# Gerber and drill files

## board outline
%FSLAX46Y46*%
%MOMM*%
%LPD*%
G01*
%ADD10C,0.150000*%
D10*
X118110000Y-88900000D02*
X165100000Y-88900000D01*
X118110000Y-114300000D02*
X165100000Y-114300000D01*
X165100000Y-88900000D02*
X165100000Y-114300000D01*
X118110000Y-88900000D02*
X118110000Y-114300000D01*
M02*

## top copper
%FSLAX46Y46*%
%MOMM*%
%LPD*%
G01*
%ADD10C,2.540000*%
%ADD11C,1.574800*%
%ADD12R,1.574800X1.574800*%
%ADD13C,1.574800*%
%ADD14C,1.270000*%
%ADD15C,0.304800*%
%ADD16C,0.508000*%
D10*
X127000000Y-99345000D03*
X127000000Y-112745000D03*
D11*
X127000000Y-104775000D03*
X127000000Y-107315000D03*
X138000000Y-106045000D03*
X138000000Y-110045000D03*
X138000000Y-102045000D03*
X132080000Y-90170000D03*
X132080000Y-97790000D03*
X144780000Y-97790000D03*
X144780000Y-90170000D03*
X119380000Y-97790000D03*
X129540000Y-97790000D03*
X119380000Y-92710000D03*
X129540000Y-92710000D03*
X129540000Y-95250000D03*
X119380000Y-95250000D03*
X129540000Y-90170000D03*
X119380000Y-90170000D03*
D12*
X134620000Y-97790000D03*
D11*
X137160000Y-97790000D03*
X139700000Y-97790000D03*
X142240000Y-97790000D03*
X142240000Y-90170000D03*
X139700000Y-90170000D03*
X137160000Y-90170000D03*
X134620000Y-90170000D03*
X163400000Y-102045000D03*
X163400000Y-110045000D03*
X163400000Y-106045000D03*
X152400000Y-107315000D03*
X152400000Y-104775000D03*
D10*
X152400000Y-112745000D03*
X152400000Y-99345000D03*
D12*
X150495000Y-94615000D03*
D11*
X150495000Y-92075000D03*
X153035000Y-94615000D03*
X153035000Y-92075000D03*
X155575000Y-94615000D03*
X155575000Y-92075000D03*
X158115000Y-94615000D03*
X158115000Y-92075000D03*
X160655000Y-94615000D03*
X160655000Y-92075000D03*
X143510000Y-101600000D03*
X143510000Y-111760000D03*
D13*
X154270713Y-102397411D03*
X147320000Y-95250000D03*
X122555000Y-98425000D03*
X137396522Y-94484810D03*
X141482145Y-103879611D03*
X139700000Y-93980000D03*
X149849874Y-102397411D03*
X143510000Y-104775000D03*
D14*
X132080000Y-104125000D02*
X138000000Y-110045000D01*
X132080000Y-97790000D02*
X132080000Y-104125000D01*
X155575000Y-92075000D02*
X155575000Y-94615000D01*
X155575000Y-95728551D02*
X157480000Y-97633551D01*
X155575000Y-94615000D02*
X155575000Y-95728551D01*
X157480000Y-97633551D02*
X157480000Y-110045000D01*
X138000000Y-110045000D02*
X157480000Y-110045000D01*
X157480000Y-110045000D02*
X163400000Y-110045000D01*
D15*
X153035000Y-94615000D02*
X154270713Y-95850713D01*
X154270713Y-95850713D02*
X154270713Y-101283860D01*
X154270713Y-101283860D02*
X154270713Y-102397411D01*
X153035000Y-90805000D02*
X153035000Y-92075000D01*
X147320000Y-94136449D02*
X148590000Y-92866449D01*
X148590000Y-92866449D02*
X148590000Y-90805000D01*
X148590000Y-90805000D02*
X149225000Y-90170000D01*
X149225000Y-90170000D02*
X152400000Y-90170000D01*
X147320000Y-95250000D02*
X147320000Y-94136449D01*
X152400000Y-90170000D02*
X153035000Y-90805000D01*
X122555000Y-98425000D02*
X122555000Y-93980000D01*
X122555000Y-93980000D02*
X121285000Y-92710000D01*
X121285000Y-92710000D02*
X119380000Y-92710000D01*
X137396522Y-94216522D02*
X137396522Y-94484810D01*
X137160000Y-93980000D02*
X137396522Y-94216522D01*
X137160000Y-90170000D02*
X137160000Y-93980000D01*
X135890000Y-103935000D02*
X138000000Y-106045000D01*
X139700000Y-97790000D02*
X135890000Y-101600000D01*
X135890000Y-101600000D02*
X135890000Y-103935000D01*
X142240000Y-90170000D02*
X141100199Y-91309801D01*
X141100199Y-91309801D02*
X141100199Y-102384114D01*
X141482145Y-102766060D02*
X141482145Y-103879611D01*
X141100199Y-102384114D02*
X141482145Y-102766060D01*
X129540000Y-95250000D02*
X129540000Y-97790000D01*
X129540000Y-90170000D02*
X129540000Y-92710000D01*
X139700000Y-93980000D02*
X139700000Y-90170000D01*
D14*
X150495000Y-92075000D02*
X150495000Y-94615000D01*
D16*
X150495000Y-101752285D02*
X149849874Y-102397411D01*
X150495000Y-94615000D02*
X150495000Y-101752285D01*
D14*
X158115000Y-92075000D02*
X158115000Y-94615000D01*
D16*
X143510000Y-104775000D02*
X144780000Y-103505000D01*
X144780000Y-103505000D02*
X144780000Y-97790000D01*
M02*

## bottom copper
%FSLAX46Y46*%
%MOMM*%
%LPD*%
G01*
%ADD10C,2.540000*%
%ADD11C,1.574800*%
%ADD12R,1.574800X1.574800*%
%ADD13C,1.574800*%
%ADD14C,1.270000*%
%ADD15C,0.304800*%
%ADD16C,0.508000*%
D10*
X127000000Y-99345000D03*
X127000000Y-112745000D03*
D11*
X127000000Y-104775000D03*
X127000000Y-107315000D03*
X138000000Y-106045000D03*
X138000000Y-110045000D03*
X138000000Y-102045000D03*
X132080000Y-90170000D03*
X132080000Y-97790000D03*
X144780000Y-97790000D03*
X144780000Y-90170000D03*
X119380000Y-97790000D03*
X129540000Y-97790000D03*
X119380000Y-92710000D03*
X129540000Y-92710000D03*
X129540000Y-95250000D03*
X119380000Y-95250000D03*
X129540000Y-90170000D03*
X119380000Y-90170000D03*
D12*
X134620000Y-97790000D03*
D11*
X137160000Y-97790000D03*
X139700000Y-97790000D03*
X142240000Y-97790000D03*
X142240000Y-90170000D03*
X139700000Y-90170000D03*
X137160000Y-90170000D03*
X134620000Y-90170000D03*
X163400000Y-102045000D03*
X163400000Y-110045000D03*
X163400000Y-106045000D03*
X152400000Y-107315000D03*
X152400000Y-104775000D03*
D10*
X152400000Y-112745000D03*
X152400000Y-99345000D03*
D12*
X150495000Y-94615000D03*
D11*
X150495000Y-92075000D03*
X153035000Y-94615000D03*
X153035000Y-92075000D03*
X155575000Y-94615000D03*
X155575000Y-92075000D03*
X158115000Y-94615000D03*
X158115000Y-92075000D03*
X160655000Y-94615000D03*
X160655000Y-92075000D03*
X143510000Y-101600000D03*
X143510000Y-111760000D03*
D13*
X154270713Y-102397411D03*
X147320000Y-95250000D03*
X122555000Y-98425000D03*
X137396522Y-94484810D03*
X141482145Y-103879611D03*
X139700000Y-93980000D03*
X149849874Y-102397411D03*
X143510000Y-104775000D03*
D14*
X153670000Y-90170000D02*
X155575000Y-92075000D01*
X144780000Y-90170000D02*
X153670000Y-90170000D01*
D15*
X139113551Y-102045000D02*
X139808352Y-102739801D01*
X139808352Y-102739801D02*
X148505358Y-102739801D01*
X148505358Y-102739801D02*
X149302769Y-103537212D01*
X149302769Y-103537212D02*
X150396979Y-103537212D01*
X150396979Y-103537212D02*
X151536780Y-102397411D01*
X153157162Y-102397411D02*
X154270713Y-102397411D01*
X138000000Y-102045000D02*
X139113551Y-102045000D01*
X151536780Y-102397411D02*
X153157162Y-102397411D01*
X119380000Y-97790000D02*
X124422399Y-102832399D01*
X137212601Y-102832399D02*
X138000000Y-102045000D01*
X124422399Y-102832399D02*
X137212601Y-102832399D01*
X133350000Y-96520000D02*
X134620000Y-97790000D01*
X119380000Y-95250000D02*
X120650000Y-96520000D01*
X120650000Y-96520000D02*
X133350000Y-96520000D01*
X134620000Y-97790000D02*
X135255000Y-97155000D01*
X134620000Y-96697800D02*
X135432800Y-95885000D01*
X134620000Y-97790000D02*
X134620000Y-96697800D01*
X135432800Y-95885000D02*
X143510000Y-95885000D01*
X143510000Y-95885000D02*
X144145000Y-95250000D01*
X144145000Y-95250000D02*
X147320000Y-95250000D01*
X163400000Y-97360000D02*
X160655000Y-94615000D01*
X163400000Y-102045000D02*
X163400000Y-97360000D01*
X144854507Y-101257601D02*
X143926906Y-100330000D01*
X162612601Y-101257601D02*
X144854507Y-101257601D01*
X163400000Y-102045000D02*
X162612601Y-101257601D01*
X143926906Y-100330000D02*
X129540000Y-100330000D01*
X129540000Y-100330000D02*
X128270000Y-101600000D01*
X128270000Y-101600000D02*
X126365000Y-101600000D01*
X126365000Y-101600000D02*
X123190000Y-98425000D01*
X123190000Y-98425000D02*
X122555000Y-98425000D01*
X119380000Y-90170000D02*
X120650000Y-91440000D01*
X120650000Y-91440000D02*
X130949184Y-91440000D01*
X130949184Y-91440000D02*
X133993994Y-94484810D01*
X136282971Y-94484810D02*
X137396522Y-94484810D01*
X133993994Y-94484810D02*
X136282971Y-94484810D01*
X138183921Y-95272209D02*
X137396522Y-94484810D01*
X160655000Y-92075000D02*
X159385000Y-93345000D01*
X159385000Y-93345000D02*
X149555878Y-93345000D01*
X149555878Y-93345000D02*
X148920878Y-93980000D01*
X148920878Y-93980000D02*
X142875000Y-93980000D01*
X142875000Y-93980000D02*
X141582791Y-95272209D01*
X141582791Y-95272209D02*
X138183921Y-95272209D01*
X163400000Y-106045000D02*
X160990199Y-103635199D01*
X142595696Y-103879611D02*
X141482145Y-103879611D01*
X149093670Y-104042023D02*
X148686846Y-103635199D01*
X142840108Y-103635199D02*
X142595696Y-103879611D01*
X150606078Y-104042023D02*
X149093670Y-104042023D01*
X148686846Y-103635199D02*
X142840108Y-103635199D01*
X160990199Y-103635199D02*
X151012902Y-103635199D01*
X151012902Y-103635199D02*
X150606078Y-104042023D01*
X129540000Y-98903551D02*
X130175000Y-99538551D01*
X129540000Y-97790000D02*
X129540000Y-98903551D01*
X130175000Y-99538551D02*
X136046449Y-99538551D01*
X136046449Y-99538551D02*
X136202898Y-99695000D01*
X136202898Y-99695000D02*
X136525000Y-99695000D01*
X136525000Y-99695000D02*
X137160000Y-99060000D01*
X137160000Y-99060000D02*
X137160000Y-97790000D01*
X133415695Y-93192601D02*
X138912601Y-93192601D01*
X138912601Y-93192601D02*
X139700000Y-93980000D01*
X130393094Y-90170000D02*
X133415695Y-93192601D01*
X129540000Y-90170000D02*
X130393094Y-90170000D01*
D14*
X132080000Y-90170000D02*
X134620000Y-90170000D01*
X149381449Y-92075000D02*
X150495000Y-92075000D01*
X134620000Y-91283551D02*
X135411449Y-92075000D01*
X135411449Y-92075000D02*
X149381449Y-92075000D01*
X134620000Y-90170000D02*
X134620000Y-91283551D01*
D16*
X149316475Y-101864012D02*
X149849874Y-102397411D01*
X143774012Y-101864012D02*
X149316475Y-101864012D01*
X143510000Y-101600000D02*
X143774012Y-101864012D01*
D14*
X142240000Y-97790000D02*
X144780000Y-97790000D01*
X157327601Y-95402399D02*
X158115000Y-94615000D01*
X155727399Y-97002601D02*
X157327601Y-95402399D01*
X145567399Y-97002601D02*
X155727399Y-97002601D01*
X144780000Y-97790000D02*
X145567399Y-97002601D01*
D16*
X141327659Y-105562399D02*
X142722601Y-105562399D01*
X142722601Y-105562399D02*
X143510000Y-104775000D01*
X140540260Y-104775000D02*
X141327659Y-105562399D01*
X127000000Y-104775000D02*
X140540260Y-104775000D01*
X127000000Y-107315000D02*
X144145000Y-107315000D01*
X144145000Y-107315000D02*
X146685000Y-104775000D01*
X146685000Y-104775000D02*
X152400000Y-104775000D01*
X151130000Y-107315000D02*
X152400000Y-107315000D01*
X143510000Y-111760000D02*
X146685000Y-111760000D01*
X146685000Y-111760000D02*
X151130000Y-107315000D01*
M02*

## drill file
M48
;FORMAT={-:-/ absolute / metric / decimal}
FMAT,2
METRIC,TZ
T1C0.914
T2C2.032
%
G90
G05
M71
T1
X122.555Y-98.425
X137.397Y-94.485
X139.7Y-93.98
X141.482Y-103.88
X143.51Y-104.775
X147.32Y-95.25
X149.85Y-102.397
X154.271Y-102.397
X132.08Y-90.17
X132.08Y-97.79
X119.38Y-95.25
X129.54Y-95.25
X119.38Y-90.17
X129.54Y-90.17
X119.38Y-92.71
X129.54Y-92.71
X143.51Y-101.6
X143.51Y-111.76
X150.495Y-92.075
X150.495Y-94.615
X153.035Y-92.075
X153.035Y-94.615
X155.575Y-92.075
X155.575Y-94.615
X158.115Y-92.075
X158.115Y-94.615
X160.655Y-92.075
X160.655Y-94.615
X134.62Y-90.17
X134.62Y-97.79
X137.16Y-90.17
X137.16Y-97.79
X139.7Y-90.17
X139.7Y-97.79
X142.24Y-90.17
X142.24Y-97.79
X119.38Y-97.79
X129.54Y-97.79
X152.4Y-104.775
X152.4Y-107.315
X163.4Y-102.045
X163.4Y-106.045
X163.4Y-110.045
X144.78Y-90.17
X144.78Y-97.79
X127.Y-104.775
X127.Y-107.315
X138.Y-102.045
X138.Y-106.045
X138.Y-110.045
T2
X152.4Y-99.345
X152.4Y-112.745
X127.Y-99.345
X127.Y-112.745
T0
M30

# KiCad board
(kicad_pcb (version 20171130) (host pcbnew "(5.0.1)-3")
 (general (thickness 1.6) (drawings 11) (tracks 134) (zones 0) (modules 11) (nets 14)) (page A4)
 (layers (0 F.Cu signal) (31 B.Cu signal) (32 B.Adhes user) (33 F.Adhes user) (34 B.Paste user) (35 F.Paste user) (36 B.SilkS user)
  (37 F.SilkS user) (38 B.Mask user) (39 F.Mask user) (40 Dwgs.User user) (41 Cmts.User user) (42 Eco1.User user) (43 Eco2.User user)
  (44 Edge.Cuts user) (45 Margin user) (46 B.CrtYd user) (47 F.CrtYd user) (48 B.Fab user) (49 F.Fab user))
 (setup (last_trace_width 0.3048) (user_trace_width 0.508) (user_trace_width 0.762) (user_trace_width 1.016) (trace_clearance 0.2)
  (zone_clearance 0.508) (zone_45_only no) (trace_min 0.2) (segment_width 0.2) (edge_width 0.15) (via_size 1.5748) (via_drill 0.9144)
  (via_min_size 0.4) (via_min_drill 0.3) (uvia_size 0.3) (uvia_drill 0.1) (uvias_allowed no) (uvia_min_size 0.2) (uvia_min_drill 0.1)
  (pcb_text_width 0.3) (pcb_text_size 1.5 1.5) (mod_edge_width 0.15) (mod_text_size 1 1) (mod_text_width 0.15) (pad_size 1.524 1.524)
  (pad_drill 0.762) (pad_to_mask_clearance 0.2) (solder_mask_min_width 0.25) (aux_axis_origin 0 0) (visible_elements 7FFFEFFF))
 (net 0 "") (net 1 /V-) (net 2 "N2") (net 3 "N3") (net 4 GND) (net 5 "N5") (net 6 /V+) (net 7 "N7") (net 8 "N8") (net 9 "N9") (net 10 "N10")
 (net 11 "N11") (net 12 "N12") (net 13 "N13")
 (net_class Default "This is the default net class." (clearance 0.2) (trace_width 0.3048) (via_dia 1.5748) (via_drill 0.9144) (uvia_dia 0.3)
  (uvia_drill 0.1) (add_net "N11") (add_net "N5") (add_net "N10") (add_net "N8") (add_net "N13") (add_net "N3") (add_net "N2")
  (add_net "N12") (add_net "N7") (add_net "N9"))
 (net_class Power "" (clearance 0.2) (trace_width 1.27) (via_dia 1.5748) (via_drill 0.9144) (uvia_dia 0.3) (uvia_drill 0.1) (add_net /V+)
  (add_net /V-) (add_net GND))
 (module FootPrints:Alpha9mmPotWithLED (layer B.Cu) (at 127 106.045 270)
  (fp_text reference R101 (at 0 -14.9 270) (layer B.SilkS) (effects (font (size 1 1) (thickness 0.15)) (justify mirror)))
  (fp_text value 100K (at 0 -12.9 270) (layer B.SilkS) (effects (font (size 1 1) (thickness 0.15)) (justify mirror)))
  (pad "" thru_hole circle (at -6.7 0 270) (size 2.54 2.54) (drill 2.032) (layers *.Cu *.Mask B.SilkS))
  (pad "" thru_hole circle (at 6.7 0 270) (size 2.54 2.54) (drill 2.032) (layers *.Cu *.Mask B.SilkS))
  (pad 4 thru_hole circle (at -1.27 0 270) (size 1.5748 1.5748) (drill 0.9144) (layers *.Cu *.Mask B.SilkS) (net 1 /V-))
  (pad 5 thru_hole circle (at 1.27 0 270) (size 1.5748 1.5748) (drill 0.9144) (layers *.Cu *.Mask B.SilkS) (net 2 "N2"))
  (pad 2 thru_hole circle (at 0 -11 270) (size 1.5748 1.5748) (drill 0.9144) (layers *.Cu *.Mask B.SilkS) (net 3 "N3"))
  (pad 3 thru_hole circle (at 4 -11 270) (size 1.5748 1.5748) (drill 0.9144) (layers *.Cu *.Mask B.SilkS) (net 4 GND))
  (pad 1 thru_hole circle (at -4 -11 270) (size 1.5748 1.5748) (drill 0.9144) (layers *.Cu *.Mask B.SilkS) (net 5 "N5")))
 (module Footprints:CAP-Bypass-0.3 (layer F.Cu) (at 132.08 93.98 270)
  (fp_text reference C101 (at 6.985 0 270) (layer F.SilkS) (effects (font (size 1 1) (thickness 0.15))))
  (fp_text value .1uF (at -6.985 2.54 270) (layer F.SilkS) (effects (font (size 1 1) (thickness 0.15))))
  (pad 1 thru_hole circle (at -3.81 0 270) (size 1.5748 1.5748) (drill 0.9144) (layers *.Cu *.Mask F.SilkS) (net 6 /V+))
  (pad 2 thru_hole circle (at 3.81 0 270) (size 1.5748 1.5748) (drill 0.9144) (layers *.Cu *.Mask F.SilkS) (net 4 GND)))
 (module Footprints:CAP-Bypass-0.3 (layer F.Cu) (at 144.78 93.98 90)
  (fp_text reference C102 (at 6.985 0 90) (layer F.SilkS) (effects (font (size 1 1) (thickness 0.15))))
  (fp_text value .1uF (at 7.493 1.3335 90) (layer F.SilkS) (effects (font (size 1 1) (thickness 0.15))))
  (pad 1 thru_hole circle (at -3.81 0 90) (size 1.5748 1.5748) (drill 0.9144) (layers *.Cu *.Mask F.SilkS) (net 1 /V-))
  (pad 2 thru_hole circle (at 3.81 0 90) (size 1.5748 1.5748) (drill 0.9144) (layers *.Cu *.Mask F.SilkS) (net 4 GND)))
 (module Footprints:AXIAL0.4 (layer F.Cu) (at 124.46 97.79)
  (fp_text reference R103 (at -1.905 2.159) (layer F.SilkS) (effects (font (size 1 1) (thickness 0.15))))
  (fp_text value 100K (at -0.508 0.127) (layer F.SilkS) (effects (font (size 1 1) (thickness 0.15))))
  (pad 1 thru_hole circle (at -5.08 0) (size 1.5748 1.5748) (drill 0.9144) (layers *.Cu *.Mask F.SilkS) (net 5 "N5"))
  (pad 2 thru_hole circle (at 5.08 0) (size 1.5748 1.5748) (drill 0.9144) (layers *.Cu *.Mask F.SilkS) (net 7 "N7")))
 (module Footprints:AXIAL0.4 (layer F.Cu) (at 124.46 92.71)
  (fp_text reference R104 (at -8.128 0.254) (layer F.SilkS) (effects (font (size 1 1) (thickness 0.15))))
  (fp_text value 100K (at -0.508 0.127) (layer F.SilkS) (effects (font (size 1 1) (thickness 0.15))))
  (pad 1 thru_hole circle (at -5.08 0) (size 1.5748 1.5748) (drill 0.9144) (layers *.Cu *.Mask F.SilkS) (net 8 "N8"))
  (pad 2 thru_hole circle (at 5.08 0) (size 1.5748 1.5748) (drill 0.9144) (layers *.Cu *.Mask F.SilkS) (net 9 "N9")))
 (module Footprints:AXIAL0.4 (layer F.Cu) (at 124.46 95.25 180)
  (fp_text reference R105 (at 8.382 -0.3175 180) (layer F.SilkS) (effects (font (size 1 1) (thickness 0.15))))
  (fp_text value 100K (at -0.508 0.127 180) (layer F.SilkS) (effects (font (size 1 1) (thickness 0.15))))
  (pad 1 thru_hole circle (at -5.08 0 180) (size 1.5748 1.5748) (drill 0.9144) (layers *.Cu *.Mask F.SilkS) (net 7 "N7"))
  (pad 2 thru_hole circle (at 5.08 0 180) (size 1.5748 1.5748) (drill 0.9144) (layers *.Cu *.Mask F.SilkS) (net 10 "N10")))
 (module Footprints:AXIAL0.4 (layer F.Cu) (at 124.46 90.17 180)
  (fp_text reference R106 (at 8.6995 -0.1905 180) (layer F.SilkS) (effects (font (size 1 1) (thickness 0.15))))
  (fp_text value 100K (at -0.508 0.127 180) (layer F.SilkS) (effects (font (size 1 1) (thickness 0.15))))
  (pad 1 thru_hole circle (at -5.08 0 180) (size 1.5748 1.5748) (drill 0.9144) (layers *.Cu *.Mask F.SilkS) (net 9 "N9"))
  (pad 2 thru_hole circle (at 5.08 0 180) (size 1.5748 1.5748) (drill 0.9144) (layers *.Cu *.Mask F.SilkS) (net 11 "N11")))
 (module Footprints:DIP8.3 (layer F.Cu) (at 138.43 93.98)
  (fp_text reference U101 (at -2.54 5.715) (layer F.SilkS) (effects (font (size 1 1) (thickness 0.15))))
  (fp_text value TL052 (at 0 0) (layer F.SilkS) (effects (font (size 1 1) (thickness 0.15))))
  (pad 1 thru_hole rect (at -3.81 3.81) (size 1.5748 1.5748) (drill 0.9144) (layers *.Cu *.Mask F.SilkS) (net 10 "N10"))
  (pad 2 thru_hole circle (at -1.27 3.81) (size 1.5748 1.5748) (drill 0.9144) (layers *.Cu *.Mask F.SilkS) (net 7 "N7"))
  (pad 3 thru_hole circle (at 1.27 3.81) (size 1.5748 1.5748) (drill 0.9144) (layers *.Cu *.Mask F.SilkS) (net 3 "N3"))
  (pad 4 thru_hole circle (at 3.81 3.81) (size 1.5748 1.5748) (drill 0.9144) (layers *.Cu *.Mask F.SilkS) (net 1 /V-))
  (pad 5 thru_hole circle (at 3.81 -3.81) (size 1.5748 1.5748) (drill 0.9144) (layers *.Cu *.Mask F.SilkS) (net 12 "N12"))
  (pad 6 thru_hole circle (at 1.27 -3.81) (size 1.5748 1.5748) (drill 0.9144) (layers *.Cu *.Mask F.SilkS) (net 9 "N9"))
  (pad 7 thru_hole circle (at -1.27 -3.81) (size 1.5748 1.5748) (drill 0.9144) (layers *.Cu *.Mask F.SilkS) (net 11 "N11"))
  (pad 8 thru_hole circle (at -3.81 -3.81) (size 1.5748 1.5748) (drill 0.9144) (layers *.Cu *.Mask F.SilkS) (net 6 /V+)))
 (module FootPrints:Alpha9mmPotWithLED (layer B.Cu) (at 152.4 106.045 270)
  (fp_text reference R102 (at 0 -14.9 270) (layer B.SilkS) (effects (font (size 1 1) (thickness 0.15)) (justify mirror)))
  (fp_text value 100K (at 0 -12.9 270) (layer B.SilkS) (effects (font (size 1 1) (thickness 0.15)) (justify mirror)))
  (pad 1 thru_hole circle (at -4 -11 270) (size 1.5748 1.5748) (drill 0.9144) (layers *.Cu *.Mask B.SilkS) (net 8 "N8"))
  (pad 3 thru_hole circle (at 4 -11 270) (size 1.5748 1.5748) (drill 0.9144) (layers *.Cu *.Mask B.SilkS) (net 4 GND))
  (pad 2 thru_hole circle (at 0 -11 270) (size 1.5748 1.5748) (drill 0.9144) (layers *.Cu *.Mask B.SilkS) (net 12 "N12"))
  (pad 5 thru_hole circle (at 1.27 0 270) (size 1.5748 1.5748) (drill 0.9144) (layers *.Cu *.Mask B.SilkS) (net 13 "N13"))
  (pad 4 thru_hole circle (at -1.27 0 270) (size 1.5748 1.5748) (drill 0.9144) (layers *.Cu *.Mask B.SilkS) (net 2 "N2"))
  (pad "" thru_hole circle (at 6.7 0 270) (size 2.54 2.54) (drill 2.032) (layers *.Cu *.Mask B.SilkS))
  (pad "" thru_hole circle (at -6.7 0 270) (size 2.54 2.54) (drill 2.032) (layers *.Cu *.Mask B.SilkS)))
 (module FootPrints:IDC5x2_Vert (layer F.Cu) (at 155.575 93.345 180)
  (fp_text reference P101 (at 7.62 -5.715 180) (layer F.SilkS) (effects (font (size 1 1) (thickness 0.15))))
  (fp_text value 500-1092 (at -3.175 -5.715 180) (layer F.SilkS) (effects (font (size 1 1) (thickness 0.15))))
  (pad 1 thru_hole rect (at 5.08 -1.27 180) (size 1.5748 1.5748) (drill 0.9144) (layers *.Cu *.Mask F.SilkS) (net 6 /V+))
  (pad 2 thru_hole circle (at 5.08 1.27 180) (size 1.5748 1.5748) (drill 0.9144) (layers *.Cu *.Mask F.SilkS) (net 6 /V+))
  (pad 3 thru_hole circle (at 2.54 -1.27 180) (size 1.5748 1.5748) (drill 0.9144) (layers *.Cu *.Mask F.SilkS) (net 5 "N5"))
  (pad 4 thru_hole circle (at 2.54 1.27 180) (size 1.5748 1.5748) (drill 0.9144) (layers *.Cu *.Mask F.SilkS) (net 10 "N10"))
  (pad 5 thru_hole circle (at 0 -1.27 180) (size 1.5748 1.5748) (drill 0.9144) (layers *.Cu *.Mask F.SilkS) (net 4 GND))
  (pad 6 thru_hole circle (at 0 1.27 180) (size 1.5748 1.5748) (drill 0.9144) (layers *.Cu *.Mask F.SilkS) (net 4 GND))
  (pad 7 thru_hole circle (at -2.54 -1.27 180) (size 1.5748 1.5748) (drill 0.9144) (layers *.Cu *.Mask F.SilkS) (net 1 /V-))
  (pad 8 thru_hole circle (at -2.54 1.27 180) (size 1.5748 1.5748) (drill 0.9144) (layers *.Cu *.Mask F.SilkS) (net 1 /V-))
  (pad 9 thru_hole circle (at -5.08 -1.27 180) (size 1.5748 1.5748) (drill 0.9144) (layers *.Cu *.Mask F.SilkS) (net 8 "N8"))
  (pad 10 thru_hole circle (at -5.08 1.27 180) (size 1.5748 1.5748) (drill 0.9144) (layers *.Cu *.Mask F.SilkS) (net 11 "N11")))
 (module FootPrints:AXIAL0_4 (layer F.Cu) (at 143.51 106.68 270)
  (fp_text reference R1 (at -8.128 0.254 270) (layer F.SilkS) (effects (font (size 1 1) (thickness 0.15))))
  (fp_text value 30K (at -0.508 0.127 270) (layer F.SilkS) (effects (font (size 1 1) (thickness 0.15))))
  (pad 1 thru_hole circle (at -5.08 0 270) (size 1.5748 1.5748) (drill 0.9144) (layers *.Cu *.Mask F.SilkS) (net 6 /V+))
  (pad 2 thru_hole circle (at 5.08 0 270) (size 1.5748 1.5748) (drill 0.9144) (layers *.Cu *.Mask F.SilkS) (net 13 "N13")))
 (gr_line (start 118.11 88.9) (end 165.1 88.9) (layer Edge.Cuts) (width 0.15))
 (gr_line (start 118.11 114.3) (end 165.1 114.3) (layer Edge.Cuts) (width 0.15))
 (gr_line (start 165.1 88.9) (end 165.1 114.3) (layer Edge.Cuts) (width 0.15))
 (gr_line (start 118.11 88.9) (end 118.11 114.3) (layer Edge.Cuts) (width 0.15))
 (segment (start 132.08 104.125) (end 138 110.045) (width 1.27) (layer F.Cu) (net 4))
 (segment (start 132.08 97.79) (end 132.08 104.125) (width 1.27) (layer F.Cu) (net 4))
 (segment (start 153.67 90.17) (end 155.575 92.075) (width 1.27) (layer B.Cu) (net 4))
 (segment (start 144.78 90.17) (end 153.67 90.17) (width 1.27) (layer B.Cu) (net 4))
 (segment (start 155.575 92.075) (end 155.575 94.615) (width 1.27) (layer F.Cu) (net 4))
 (segment (start 155.575 95.728551) (end 157.48 97.633551) (width 1.27) (layer F.Cu) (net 4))
 (segment (start 155.575 94.615) (end 155.575 95.728551) (width 1.27) (layer F.Cu) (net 4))
 (segment (start 157.48 97.633551) (end 157.48 110.045) (width 1.27) (layer F.Cu) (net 4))
 (segment (start 138 110.045) (end 157.48 110.045) (width 1.27) (layer F.Cu) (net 4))
 (segment (start 157.48 110.045) (end 163.4 110.045) (width 1.27) (layer F.Cu) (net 4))
 (segment (start 139.113551 102.045) (end 139.808352 102.739801) (width 0.3048) (layer B.Cu) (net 5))
 (segment (start 139.808352 102.739801) (end 148.505358 102.739801) (width 0.3048) (layer B.Cu) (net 5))
 (segment (start 148.505358 102.739801) (end 149.302769 103.537212) (width 0.3048) (layer B.Cu) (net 5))
 (segment (start 149.302769 103.537212) (end 150.396979 103.537212) (width 0.3048) (layer B.Cu) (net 5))
 (segment (start 150.396979 103.537212) (end 151.53678 102.397411) (width 0.3048) (layer B.Cu) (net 5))
 (via (at 154.270713 102.397411) (size 1.5748) (drill 0.9144) (layers F.Cu B.Cu) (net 5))
 (segment (start 153.035 94.615) (end 154.270713 95.850713) (width 0.3048) (layer F.Cu) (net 5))
 (segment (start 154.270713 95.850713) (end 154.270713 101.28386) (width 0.3048) (layer F.Cu) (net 5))
 (segment (start 153.157162 102.397411) (end 154.270713 102.397411) (width 0.3048) (layer B.Cu) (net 5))
 (segment (start 138 102.045) (end 139.113551 102.045) (width 0.3048) (layer B.Cu) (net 5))
 (segment (start 154.270713 101.28386) (end 154.270713 102.397411) (width 0.3048) (layer F.Cu) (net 5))
 (segment (start 151.53678 102.397411) (end 153.157162 102.397411) (width 0.3048) (layer B.Cu) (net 5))
 (segment (start 119.38 97.79) (end 124.422399 102.832399) (width 0.3048) (layer B.Cu) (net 5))
 (segment (start 137.212601 102.832399) (end 138 102.045) (width 0.3048) (layer B.Cu) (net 5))
 (segment (start 124.422399 102.832399) (end 137.212601 102.832399) (width 0.3048) (layer B.Cu) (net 5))
 (segment (start 133.35 96.52) (end 134.62 97.79) (width 0.3048) (layer B.Cu) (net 10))
 (segment (start 119.38 95.25) (end 120.65 96.52) (width 0.3048) (layer B.Cu) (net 10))
 (segment (start 120.65 96.52) (end 133.35 96.52) (width 0.3048) (layer B.Cu) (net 10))
 (segment (start 134.62 97.79) (end 135.255 97.155) (width 0.3048) (layer B.Cu) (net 10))
 (segment (start 134.62 96.6978) (end 135.4328 95.885) (width 0.3048) (layer B.Cu) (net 10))
 (segment (start 134.62 97.79) (end 134.62 96.6978) (width 0.3048) (layer B.Cu) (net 10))
 (segment (start 135.4328 95.885) (end 143.51 95.885) (width 0.3048) (layer B.Cu) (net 10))
 (via (at 147.32 95.25) (size 1.5748) (drill 0.9144) (layers F.Cu B.Cu) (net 10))
 (segment (start 143.51 95.885) (end 144.145 95.25) (width 0.3048) (layer B.Cu) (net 10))
 (segment (start 144.145 95.25) (end 147.32 95.25) (width 0.3048) (layer B.Cu) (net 10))
 (segment (start 153.035 90.805) (end 153.035 92.075) (width 0.3048) (layer F.Cu) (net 10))
 (segment (start 147.32 94.136449) (end 148.59 92.866449) (width 0.3048) (layer F.Cu) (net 10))
 (segment (start 148.59 92.866449) (end 148.59 90.805) (width 0.3048) (layer F.Cu) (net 10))
 (segment (start 148.59 90.805) (end 149.225 90.17) (width 0.3048) (layer F.Cu) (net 10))
 (segment (start 149.225 90.17) (end 152.4 90.17) (width 0.3048) (layer F.Cu) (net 10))
 (segment (start 147.32 95.25) (end 147.32 94.136449) (width 0.3048) (layer F.Cu) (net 10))
 (segment (start 152.4 90.17) (end 153.035 90.805) (width 0.3048) (layer F.Cu) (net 10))
 (segment (start 163.4 97.36) (end 160.655 94.615) (width 0.3048) (layer B.Cu) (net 8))
 (segment (start 163.4 102.045) (end 163.4 97.36) (width 0.3048) (layer B.Cu) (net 8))
 (segment (start 144.854507 101.257601) (end 143.926906 100.33) (width 0.3048) (layer B.Cu) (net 8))
 (segment (start 162.612601 101.257601) (end 144.854507 101.257601) (width 0.3048) (layer B.Cu) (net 8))
 (segment (start 163.4 102.045) (end 162.612601 101.257601) (width 0.3048) (layer B.Cu) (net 8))
 (segment (start 143.926906 100.33) (end 129.54 100.33) (width 0.3048) (layer B.Cu) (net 8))
 (segment (start 129.54 100.33) (end 128.27 101.6) (width 0.3048) (layer B.Cu) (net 8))
 (segment (start 128.27 101.6) (end 126.365 101.6) (width 0.3048) (layer B.Cu) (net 8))
 (via (at 122.555 98.425) (size 1.5748) (drill 0.9144) (layers F.Cu B.Cu) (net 8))
 (segment (start 126.365 101.6) (end 123.19 98.425) (width 0.3048) (layer B.Cu) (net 8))
 (segment (start 123.19 98.425) (end 122.555 98.425) (width 0.3048) (layer B.Cu) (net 8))
 (segment (start 122.555 98.425) (end 122.555 93.98) (width 0.3048) (layer F.Cu) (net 8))
 (segment (start 122.555 93.98) (end 121.285 92.71) (width 0.3048) (layer F.Cu) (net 8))
 (segment (start 121.285 92.71) (end 119.38 92.71) (width 0.3048) (layer F.Cu) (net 8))
 (segment (start 137.396522 94.216522) (end 137.396522 94.48481) (width 0.3048) (layer F.Cu) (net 11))
 (segment (start 137.16 93.98) (end 137.396522 94.216522) (width 0.3048) (layer F.Cu) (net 11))
 (segment (start 119.38 90.17) (end 120.65 91.44) (width 0.3048) (layer B.Cu) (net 11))
 (segment (start 120.65 91.44) (end 130.949184 91.44) (width 0.3048) (layer B.Cu) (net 11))
 (segment (start 130.949184 91.44) (end 133.993994 94.48481) (width 0.3048) (layer B.Cu) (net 11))
 (segment (start 136.282971 94.48481) (end 137.396522 94.48481) (width 0.3048) (layer B.Cu) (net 11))
 (segment (start 137.16 90.17) (end 137.16 93.98) (width 0.3048) (layer F.Cu) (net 11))
 (segment (start 133.993994 94.48481) (end 136.282971 94.48481) (width 0.3048) (layer B.Cu) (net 11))
 (via (at 137.396522 94.48481) (size 1.5748) (drill 0.9144) (layers F.Cu B.Cu) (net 11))
 (segment (start 138.183921 95.272209) (end 137.396522 94.48481) (width 0.3048) (layer B.Cu) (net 11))
 (segment (start 160.655 92.075) (end 159.385 93.345) (width 0.3048) (layer B.Cu) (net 11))
 (segment (start 159.385 93.345) (end 149.555878 93.345) (width 0.3048) (layer B.Cu) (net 11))
 (segment (start 149.555878 93.345) (end 148.920878 93.98) (width 0.3048) (layer B.Cu) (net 11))
 (segment (start 148.920878 93.98) (end 142.875 93.98) (width 0.3048) (layer B.Cu) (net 11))
 (segment (start 142.875 93.98) (end 141.582791 95.272209) (width 0.3048) (layer B.Cu) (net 11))
 (segment (start 141.582791 95.272209) (end 138.183921 95.272209) (width 0.3048) (layer B.Cu) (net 11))
 (segment (start 135.89 103.935) (end 138 106.045) (width 0.3048) (layer F.Cu) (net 3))
 (segment (start 139.7 97.79) (end 135.89 101.6) (width 0.3048) (layer F.Cu) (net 3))
 (segment (start 135.89 101.6) (end 135.89 103.935) (width 0.3048) (layer F.Cu) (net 3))
 (via (at 141.482145 103.879611) (size 1.5748) (drill 0.9144) (layers F.Cu B.Cu) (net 12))
 (segment (start 142.24 90.17) (end 141.100199 91.309801) (width 0.3048) (layer F.Cu) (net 12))
 (segment (start 141.100199 91.309801) (end 141.100199 102.384114) (width 0.3048) (layer F.Cu) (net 12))
 (segment (start 141.482145 102.76606) (end 141.482145 103.879611) (width 0.3048) (layer F.Cu) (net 12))
 (segment (start 141.100199 102.384114) (end 141.482145 102.76606) (width 0.3048) (layer F.Cu) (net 12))
 (segment (start 163.4 106.045) (end 160.990199 103.635199) (width 0.3048) (layer B.Cu) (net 12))
 (segment (start 142.595696 103.879611) (end 141.482145 103.879611) (width 0.3048) (layer B.Cu) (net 12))
 (segment (start 149.09367 104.042023) (end 148.686846 103.635199) (width 0.3048) (layer B.Cu) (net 12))
 (segment (start 142.840108 103.635199) (end 142.595696 103.879611) (width 0.3048) (layer B.Cu) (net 12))
 (segment (start 150.606078 104.042023) (end 149.09367 104.042023) (width 0.3048) (layer B.Cu) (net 12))
 (segment (start 148.686846 103.635199) (end 142.840108 103.635199) (width 0.3048) (layer B.Cu) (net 12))
 (segment (start 160.990199 103.635199) (end 151.012902 103.635199) (width 0.3048) (layer B.Cu) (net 12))
 (segment (start 151.012902 103.635199) (end 150.606078 104.042023) (width 0.3048) (layer B.Cu) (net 12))
 (segment (start 129.54 95.25) (end 129.54 97.79) (width 0.3048) (layer F.Cu) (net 7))
 (segment (start 129.54 98.903551) (end 130.175 99.538551) (width 0.3048) (layer B.Cu) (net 7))
 (segment (start 129.54 97.79) (end 129.54 98.903551) (width 0.3048) (layer B.Cu) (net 7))
 (segment (start 130.175 99.538551) (end 136.046449 99.538551) (width 0.3048) (layer B.Cu) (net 7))
 (segment (start 136.046449 99.538551) (end 136.202898 99.695) (width 0.3048) (layer B.Cu) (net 7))
 (segment (start 136.202898 99.695) (end 136.525 99.695) (width 0.3048) (layer B.Cu) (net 7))
 (segment (start 136.525 99.695) (end 137.16 99.06) (width 0.3048) (layer B.Cu) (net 7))
 (segment (start 137.16 99.06) (end 137.16 97.79) (width 0.3048) (layer B.Cu) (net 7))
 (segment (start 129.54 90.17) (end 129.54 92.71) (width 0.3048) (layer F.Cu) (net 9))
 (via (at 139.7 93.98) (size 1.5748) (drill 0.9144) (layers F.Cu B.Cu) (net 9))
 (segment (start 139.7 93.98) (end 139.7 90.17) (width 0.3048) (layer F.Cu) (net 9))
 (segment (start 133.415695 93.192601) (end 138.912601 93.192601) (width 0.3048) (layer B.Cu) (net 9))
 (segment (start 138.912601 93.192601) (end 139.7 93.98) (width 0.3048) (layer B.Cu) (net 9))
 (segment (start 130.393094 90.17) (end 133.415695 93.192601) (width 0.3048) (layer B.Cu) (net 9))
 (segment (start 129.54 90.17) (end 130.393094 90.17) (width 0.3048) (layer B.Cu) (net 9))
 (segment (start 132.08 90.17) (end 134.62 90.17) (width 1.27) (layer B.Cu) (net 6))
 (segment (start 149.381449 92.075) (end 150.495 92.075) (width 1.27) (layer B.Cu) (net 6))
 (segment (start 134.62 91.283551) (end 135.411449 92.075) (width 1.27) (layer B.Cu) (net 6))
 (segment (start 135.411449 92.075) (end 149.381449 92.075) (width 1.27) (layer B.Cu) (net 6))
 (segment (start 134.62 90.17) (end 134.62 91.283551) (width 1.27) (layer B.Cu) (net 6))
 (segment (start 150.495 92.075) (end 150.495 94.615) (width 1.27) (layer F.Cu) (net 6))
 (segment (start 149.316475 101.864012) (end 149.849874 102.397411) (width 0.508) (layer B.Cu) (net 6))
 (via (at 149.849874 102.397411) (size 1.5748) (drill 0.9144) (layers F.Cu B.Cu) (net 6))
 (segment (start 150.495 101.752285) (end 149.849874 102.397411) (width 0.508) (layer F.Cu) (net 6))
 (segment (start 143.774012 101.864012) (end 149.316475 101.864012) (width 0.508) (layer B.Cu) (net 6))
 (segment (start 143.51 101.6) (end 143.774012 101.864012) (width 0.508) (layer B.Cu) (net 6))
 (segment (start 150.495 94.615) (end 150.495 101.752285) (width 0.508) (layer F.Cu) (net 6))
 (segment (start 142.24 97.79) (end 144.78 97.79) (width 1.27) (layer B.Cu) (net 1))
 (segment (start 158.115 92.075) (end 158.115 94.615) (width 1.27) (layer F.Cu) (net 1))
 (via (at 143.51 104.775) (size 1.5748) (drill 0.9144) (layers F.Cu B.Cu) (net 1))
 (segment (start 143.51 104.775) (end 144.78 103.505) (width 0.508) (layer F.Cu) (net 1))
 (segment (start 144.78 103.505) (end 144.78 97.79) (width 0.508) (layer F.Cu) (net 1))
 (segment (start 157.327601 95.402399) (end 158.115 94.615) (width 1.27) (layer B.Cu) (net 1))
 (segment (start 155.727399 97.002601) (end 157.327601 95.402399) (width 1.27) (layer B.Cu) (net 1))
 (segment (start 145.567399 97.002601) (end 155.727399 97.002601) (width 1.27) (layer B.Cu) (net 1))
 (segment (start 144.78 97.79) (end 145.567399 97.002601) (width 1.27) (layer B.Cu) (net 1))
 (segment (start 141.327659 105.562399) (end 142.722601 105.562399) (width 0.508) (layer B.Cu) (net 1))
 (segment (start 142.722601 105.562399) (end 143.51 104.775) (width 0.508) (layer B.Cu) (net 1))
 (segment (start 140.54026 104.775) (end 141.327659 105.562399) (width 0.508) (layer B.Cu) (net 1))
 (segment (start 127 104.775) (end 140.54026 104.775) (width 0.508) (layer B.Cu) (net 1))
 (segment (start 127 107.315) (end 144.145 107.315) (width 0.508) (layer B.Cu) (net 2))
 (segment (start 144.145 107.315) (end 146.685 104.775) (width 0.508) (layer B.Cu) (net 2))
 (segment (start 146.685 104.775) (end 152.4 104.775) (width 0.508) (layer B.Cu) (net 2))
 (segment (start 151.13 107.315) (end 152.4 107.315) (width 0.508) (layer B.Cu) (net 13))
 (segment (start 143.51 111.76) (end 146.685 111.76) (width 0.508) (layer B.Cu) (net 13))
 (segment (start 146.685 111.76) (end 151.13 107.315) (width 0.508) (layer B.Cu) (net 13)))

